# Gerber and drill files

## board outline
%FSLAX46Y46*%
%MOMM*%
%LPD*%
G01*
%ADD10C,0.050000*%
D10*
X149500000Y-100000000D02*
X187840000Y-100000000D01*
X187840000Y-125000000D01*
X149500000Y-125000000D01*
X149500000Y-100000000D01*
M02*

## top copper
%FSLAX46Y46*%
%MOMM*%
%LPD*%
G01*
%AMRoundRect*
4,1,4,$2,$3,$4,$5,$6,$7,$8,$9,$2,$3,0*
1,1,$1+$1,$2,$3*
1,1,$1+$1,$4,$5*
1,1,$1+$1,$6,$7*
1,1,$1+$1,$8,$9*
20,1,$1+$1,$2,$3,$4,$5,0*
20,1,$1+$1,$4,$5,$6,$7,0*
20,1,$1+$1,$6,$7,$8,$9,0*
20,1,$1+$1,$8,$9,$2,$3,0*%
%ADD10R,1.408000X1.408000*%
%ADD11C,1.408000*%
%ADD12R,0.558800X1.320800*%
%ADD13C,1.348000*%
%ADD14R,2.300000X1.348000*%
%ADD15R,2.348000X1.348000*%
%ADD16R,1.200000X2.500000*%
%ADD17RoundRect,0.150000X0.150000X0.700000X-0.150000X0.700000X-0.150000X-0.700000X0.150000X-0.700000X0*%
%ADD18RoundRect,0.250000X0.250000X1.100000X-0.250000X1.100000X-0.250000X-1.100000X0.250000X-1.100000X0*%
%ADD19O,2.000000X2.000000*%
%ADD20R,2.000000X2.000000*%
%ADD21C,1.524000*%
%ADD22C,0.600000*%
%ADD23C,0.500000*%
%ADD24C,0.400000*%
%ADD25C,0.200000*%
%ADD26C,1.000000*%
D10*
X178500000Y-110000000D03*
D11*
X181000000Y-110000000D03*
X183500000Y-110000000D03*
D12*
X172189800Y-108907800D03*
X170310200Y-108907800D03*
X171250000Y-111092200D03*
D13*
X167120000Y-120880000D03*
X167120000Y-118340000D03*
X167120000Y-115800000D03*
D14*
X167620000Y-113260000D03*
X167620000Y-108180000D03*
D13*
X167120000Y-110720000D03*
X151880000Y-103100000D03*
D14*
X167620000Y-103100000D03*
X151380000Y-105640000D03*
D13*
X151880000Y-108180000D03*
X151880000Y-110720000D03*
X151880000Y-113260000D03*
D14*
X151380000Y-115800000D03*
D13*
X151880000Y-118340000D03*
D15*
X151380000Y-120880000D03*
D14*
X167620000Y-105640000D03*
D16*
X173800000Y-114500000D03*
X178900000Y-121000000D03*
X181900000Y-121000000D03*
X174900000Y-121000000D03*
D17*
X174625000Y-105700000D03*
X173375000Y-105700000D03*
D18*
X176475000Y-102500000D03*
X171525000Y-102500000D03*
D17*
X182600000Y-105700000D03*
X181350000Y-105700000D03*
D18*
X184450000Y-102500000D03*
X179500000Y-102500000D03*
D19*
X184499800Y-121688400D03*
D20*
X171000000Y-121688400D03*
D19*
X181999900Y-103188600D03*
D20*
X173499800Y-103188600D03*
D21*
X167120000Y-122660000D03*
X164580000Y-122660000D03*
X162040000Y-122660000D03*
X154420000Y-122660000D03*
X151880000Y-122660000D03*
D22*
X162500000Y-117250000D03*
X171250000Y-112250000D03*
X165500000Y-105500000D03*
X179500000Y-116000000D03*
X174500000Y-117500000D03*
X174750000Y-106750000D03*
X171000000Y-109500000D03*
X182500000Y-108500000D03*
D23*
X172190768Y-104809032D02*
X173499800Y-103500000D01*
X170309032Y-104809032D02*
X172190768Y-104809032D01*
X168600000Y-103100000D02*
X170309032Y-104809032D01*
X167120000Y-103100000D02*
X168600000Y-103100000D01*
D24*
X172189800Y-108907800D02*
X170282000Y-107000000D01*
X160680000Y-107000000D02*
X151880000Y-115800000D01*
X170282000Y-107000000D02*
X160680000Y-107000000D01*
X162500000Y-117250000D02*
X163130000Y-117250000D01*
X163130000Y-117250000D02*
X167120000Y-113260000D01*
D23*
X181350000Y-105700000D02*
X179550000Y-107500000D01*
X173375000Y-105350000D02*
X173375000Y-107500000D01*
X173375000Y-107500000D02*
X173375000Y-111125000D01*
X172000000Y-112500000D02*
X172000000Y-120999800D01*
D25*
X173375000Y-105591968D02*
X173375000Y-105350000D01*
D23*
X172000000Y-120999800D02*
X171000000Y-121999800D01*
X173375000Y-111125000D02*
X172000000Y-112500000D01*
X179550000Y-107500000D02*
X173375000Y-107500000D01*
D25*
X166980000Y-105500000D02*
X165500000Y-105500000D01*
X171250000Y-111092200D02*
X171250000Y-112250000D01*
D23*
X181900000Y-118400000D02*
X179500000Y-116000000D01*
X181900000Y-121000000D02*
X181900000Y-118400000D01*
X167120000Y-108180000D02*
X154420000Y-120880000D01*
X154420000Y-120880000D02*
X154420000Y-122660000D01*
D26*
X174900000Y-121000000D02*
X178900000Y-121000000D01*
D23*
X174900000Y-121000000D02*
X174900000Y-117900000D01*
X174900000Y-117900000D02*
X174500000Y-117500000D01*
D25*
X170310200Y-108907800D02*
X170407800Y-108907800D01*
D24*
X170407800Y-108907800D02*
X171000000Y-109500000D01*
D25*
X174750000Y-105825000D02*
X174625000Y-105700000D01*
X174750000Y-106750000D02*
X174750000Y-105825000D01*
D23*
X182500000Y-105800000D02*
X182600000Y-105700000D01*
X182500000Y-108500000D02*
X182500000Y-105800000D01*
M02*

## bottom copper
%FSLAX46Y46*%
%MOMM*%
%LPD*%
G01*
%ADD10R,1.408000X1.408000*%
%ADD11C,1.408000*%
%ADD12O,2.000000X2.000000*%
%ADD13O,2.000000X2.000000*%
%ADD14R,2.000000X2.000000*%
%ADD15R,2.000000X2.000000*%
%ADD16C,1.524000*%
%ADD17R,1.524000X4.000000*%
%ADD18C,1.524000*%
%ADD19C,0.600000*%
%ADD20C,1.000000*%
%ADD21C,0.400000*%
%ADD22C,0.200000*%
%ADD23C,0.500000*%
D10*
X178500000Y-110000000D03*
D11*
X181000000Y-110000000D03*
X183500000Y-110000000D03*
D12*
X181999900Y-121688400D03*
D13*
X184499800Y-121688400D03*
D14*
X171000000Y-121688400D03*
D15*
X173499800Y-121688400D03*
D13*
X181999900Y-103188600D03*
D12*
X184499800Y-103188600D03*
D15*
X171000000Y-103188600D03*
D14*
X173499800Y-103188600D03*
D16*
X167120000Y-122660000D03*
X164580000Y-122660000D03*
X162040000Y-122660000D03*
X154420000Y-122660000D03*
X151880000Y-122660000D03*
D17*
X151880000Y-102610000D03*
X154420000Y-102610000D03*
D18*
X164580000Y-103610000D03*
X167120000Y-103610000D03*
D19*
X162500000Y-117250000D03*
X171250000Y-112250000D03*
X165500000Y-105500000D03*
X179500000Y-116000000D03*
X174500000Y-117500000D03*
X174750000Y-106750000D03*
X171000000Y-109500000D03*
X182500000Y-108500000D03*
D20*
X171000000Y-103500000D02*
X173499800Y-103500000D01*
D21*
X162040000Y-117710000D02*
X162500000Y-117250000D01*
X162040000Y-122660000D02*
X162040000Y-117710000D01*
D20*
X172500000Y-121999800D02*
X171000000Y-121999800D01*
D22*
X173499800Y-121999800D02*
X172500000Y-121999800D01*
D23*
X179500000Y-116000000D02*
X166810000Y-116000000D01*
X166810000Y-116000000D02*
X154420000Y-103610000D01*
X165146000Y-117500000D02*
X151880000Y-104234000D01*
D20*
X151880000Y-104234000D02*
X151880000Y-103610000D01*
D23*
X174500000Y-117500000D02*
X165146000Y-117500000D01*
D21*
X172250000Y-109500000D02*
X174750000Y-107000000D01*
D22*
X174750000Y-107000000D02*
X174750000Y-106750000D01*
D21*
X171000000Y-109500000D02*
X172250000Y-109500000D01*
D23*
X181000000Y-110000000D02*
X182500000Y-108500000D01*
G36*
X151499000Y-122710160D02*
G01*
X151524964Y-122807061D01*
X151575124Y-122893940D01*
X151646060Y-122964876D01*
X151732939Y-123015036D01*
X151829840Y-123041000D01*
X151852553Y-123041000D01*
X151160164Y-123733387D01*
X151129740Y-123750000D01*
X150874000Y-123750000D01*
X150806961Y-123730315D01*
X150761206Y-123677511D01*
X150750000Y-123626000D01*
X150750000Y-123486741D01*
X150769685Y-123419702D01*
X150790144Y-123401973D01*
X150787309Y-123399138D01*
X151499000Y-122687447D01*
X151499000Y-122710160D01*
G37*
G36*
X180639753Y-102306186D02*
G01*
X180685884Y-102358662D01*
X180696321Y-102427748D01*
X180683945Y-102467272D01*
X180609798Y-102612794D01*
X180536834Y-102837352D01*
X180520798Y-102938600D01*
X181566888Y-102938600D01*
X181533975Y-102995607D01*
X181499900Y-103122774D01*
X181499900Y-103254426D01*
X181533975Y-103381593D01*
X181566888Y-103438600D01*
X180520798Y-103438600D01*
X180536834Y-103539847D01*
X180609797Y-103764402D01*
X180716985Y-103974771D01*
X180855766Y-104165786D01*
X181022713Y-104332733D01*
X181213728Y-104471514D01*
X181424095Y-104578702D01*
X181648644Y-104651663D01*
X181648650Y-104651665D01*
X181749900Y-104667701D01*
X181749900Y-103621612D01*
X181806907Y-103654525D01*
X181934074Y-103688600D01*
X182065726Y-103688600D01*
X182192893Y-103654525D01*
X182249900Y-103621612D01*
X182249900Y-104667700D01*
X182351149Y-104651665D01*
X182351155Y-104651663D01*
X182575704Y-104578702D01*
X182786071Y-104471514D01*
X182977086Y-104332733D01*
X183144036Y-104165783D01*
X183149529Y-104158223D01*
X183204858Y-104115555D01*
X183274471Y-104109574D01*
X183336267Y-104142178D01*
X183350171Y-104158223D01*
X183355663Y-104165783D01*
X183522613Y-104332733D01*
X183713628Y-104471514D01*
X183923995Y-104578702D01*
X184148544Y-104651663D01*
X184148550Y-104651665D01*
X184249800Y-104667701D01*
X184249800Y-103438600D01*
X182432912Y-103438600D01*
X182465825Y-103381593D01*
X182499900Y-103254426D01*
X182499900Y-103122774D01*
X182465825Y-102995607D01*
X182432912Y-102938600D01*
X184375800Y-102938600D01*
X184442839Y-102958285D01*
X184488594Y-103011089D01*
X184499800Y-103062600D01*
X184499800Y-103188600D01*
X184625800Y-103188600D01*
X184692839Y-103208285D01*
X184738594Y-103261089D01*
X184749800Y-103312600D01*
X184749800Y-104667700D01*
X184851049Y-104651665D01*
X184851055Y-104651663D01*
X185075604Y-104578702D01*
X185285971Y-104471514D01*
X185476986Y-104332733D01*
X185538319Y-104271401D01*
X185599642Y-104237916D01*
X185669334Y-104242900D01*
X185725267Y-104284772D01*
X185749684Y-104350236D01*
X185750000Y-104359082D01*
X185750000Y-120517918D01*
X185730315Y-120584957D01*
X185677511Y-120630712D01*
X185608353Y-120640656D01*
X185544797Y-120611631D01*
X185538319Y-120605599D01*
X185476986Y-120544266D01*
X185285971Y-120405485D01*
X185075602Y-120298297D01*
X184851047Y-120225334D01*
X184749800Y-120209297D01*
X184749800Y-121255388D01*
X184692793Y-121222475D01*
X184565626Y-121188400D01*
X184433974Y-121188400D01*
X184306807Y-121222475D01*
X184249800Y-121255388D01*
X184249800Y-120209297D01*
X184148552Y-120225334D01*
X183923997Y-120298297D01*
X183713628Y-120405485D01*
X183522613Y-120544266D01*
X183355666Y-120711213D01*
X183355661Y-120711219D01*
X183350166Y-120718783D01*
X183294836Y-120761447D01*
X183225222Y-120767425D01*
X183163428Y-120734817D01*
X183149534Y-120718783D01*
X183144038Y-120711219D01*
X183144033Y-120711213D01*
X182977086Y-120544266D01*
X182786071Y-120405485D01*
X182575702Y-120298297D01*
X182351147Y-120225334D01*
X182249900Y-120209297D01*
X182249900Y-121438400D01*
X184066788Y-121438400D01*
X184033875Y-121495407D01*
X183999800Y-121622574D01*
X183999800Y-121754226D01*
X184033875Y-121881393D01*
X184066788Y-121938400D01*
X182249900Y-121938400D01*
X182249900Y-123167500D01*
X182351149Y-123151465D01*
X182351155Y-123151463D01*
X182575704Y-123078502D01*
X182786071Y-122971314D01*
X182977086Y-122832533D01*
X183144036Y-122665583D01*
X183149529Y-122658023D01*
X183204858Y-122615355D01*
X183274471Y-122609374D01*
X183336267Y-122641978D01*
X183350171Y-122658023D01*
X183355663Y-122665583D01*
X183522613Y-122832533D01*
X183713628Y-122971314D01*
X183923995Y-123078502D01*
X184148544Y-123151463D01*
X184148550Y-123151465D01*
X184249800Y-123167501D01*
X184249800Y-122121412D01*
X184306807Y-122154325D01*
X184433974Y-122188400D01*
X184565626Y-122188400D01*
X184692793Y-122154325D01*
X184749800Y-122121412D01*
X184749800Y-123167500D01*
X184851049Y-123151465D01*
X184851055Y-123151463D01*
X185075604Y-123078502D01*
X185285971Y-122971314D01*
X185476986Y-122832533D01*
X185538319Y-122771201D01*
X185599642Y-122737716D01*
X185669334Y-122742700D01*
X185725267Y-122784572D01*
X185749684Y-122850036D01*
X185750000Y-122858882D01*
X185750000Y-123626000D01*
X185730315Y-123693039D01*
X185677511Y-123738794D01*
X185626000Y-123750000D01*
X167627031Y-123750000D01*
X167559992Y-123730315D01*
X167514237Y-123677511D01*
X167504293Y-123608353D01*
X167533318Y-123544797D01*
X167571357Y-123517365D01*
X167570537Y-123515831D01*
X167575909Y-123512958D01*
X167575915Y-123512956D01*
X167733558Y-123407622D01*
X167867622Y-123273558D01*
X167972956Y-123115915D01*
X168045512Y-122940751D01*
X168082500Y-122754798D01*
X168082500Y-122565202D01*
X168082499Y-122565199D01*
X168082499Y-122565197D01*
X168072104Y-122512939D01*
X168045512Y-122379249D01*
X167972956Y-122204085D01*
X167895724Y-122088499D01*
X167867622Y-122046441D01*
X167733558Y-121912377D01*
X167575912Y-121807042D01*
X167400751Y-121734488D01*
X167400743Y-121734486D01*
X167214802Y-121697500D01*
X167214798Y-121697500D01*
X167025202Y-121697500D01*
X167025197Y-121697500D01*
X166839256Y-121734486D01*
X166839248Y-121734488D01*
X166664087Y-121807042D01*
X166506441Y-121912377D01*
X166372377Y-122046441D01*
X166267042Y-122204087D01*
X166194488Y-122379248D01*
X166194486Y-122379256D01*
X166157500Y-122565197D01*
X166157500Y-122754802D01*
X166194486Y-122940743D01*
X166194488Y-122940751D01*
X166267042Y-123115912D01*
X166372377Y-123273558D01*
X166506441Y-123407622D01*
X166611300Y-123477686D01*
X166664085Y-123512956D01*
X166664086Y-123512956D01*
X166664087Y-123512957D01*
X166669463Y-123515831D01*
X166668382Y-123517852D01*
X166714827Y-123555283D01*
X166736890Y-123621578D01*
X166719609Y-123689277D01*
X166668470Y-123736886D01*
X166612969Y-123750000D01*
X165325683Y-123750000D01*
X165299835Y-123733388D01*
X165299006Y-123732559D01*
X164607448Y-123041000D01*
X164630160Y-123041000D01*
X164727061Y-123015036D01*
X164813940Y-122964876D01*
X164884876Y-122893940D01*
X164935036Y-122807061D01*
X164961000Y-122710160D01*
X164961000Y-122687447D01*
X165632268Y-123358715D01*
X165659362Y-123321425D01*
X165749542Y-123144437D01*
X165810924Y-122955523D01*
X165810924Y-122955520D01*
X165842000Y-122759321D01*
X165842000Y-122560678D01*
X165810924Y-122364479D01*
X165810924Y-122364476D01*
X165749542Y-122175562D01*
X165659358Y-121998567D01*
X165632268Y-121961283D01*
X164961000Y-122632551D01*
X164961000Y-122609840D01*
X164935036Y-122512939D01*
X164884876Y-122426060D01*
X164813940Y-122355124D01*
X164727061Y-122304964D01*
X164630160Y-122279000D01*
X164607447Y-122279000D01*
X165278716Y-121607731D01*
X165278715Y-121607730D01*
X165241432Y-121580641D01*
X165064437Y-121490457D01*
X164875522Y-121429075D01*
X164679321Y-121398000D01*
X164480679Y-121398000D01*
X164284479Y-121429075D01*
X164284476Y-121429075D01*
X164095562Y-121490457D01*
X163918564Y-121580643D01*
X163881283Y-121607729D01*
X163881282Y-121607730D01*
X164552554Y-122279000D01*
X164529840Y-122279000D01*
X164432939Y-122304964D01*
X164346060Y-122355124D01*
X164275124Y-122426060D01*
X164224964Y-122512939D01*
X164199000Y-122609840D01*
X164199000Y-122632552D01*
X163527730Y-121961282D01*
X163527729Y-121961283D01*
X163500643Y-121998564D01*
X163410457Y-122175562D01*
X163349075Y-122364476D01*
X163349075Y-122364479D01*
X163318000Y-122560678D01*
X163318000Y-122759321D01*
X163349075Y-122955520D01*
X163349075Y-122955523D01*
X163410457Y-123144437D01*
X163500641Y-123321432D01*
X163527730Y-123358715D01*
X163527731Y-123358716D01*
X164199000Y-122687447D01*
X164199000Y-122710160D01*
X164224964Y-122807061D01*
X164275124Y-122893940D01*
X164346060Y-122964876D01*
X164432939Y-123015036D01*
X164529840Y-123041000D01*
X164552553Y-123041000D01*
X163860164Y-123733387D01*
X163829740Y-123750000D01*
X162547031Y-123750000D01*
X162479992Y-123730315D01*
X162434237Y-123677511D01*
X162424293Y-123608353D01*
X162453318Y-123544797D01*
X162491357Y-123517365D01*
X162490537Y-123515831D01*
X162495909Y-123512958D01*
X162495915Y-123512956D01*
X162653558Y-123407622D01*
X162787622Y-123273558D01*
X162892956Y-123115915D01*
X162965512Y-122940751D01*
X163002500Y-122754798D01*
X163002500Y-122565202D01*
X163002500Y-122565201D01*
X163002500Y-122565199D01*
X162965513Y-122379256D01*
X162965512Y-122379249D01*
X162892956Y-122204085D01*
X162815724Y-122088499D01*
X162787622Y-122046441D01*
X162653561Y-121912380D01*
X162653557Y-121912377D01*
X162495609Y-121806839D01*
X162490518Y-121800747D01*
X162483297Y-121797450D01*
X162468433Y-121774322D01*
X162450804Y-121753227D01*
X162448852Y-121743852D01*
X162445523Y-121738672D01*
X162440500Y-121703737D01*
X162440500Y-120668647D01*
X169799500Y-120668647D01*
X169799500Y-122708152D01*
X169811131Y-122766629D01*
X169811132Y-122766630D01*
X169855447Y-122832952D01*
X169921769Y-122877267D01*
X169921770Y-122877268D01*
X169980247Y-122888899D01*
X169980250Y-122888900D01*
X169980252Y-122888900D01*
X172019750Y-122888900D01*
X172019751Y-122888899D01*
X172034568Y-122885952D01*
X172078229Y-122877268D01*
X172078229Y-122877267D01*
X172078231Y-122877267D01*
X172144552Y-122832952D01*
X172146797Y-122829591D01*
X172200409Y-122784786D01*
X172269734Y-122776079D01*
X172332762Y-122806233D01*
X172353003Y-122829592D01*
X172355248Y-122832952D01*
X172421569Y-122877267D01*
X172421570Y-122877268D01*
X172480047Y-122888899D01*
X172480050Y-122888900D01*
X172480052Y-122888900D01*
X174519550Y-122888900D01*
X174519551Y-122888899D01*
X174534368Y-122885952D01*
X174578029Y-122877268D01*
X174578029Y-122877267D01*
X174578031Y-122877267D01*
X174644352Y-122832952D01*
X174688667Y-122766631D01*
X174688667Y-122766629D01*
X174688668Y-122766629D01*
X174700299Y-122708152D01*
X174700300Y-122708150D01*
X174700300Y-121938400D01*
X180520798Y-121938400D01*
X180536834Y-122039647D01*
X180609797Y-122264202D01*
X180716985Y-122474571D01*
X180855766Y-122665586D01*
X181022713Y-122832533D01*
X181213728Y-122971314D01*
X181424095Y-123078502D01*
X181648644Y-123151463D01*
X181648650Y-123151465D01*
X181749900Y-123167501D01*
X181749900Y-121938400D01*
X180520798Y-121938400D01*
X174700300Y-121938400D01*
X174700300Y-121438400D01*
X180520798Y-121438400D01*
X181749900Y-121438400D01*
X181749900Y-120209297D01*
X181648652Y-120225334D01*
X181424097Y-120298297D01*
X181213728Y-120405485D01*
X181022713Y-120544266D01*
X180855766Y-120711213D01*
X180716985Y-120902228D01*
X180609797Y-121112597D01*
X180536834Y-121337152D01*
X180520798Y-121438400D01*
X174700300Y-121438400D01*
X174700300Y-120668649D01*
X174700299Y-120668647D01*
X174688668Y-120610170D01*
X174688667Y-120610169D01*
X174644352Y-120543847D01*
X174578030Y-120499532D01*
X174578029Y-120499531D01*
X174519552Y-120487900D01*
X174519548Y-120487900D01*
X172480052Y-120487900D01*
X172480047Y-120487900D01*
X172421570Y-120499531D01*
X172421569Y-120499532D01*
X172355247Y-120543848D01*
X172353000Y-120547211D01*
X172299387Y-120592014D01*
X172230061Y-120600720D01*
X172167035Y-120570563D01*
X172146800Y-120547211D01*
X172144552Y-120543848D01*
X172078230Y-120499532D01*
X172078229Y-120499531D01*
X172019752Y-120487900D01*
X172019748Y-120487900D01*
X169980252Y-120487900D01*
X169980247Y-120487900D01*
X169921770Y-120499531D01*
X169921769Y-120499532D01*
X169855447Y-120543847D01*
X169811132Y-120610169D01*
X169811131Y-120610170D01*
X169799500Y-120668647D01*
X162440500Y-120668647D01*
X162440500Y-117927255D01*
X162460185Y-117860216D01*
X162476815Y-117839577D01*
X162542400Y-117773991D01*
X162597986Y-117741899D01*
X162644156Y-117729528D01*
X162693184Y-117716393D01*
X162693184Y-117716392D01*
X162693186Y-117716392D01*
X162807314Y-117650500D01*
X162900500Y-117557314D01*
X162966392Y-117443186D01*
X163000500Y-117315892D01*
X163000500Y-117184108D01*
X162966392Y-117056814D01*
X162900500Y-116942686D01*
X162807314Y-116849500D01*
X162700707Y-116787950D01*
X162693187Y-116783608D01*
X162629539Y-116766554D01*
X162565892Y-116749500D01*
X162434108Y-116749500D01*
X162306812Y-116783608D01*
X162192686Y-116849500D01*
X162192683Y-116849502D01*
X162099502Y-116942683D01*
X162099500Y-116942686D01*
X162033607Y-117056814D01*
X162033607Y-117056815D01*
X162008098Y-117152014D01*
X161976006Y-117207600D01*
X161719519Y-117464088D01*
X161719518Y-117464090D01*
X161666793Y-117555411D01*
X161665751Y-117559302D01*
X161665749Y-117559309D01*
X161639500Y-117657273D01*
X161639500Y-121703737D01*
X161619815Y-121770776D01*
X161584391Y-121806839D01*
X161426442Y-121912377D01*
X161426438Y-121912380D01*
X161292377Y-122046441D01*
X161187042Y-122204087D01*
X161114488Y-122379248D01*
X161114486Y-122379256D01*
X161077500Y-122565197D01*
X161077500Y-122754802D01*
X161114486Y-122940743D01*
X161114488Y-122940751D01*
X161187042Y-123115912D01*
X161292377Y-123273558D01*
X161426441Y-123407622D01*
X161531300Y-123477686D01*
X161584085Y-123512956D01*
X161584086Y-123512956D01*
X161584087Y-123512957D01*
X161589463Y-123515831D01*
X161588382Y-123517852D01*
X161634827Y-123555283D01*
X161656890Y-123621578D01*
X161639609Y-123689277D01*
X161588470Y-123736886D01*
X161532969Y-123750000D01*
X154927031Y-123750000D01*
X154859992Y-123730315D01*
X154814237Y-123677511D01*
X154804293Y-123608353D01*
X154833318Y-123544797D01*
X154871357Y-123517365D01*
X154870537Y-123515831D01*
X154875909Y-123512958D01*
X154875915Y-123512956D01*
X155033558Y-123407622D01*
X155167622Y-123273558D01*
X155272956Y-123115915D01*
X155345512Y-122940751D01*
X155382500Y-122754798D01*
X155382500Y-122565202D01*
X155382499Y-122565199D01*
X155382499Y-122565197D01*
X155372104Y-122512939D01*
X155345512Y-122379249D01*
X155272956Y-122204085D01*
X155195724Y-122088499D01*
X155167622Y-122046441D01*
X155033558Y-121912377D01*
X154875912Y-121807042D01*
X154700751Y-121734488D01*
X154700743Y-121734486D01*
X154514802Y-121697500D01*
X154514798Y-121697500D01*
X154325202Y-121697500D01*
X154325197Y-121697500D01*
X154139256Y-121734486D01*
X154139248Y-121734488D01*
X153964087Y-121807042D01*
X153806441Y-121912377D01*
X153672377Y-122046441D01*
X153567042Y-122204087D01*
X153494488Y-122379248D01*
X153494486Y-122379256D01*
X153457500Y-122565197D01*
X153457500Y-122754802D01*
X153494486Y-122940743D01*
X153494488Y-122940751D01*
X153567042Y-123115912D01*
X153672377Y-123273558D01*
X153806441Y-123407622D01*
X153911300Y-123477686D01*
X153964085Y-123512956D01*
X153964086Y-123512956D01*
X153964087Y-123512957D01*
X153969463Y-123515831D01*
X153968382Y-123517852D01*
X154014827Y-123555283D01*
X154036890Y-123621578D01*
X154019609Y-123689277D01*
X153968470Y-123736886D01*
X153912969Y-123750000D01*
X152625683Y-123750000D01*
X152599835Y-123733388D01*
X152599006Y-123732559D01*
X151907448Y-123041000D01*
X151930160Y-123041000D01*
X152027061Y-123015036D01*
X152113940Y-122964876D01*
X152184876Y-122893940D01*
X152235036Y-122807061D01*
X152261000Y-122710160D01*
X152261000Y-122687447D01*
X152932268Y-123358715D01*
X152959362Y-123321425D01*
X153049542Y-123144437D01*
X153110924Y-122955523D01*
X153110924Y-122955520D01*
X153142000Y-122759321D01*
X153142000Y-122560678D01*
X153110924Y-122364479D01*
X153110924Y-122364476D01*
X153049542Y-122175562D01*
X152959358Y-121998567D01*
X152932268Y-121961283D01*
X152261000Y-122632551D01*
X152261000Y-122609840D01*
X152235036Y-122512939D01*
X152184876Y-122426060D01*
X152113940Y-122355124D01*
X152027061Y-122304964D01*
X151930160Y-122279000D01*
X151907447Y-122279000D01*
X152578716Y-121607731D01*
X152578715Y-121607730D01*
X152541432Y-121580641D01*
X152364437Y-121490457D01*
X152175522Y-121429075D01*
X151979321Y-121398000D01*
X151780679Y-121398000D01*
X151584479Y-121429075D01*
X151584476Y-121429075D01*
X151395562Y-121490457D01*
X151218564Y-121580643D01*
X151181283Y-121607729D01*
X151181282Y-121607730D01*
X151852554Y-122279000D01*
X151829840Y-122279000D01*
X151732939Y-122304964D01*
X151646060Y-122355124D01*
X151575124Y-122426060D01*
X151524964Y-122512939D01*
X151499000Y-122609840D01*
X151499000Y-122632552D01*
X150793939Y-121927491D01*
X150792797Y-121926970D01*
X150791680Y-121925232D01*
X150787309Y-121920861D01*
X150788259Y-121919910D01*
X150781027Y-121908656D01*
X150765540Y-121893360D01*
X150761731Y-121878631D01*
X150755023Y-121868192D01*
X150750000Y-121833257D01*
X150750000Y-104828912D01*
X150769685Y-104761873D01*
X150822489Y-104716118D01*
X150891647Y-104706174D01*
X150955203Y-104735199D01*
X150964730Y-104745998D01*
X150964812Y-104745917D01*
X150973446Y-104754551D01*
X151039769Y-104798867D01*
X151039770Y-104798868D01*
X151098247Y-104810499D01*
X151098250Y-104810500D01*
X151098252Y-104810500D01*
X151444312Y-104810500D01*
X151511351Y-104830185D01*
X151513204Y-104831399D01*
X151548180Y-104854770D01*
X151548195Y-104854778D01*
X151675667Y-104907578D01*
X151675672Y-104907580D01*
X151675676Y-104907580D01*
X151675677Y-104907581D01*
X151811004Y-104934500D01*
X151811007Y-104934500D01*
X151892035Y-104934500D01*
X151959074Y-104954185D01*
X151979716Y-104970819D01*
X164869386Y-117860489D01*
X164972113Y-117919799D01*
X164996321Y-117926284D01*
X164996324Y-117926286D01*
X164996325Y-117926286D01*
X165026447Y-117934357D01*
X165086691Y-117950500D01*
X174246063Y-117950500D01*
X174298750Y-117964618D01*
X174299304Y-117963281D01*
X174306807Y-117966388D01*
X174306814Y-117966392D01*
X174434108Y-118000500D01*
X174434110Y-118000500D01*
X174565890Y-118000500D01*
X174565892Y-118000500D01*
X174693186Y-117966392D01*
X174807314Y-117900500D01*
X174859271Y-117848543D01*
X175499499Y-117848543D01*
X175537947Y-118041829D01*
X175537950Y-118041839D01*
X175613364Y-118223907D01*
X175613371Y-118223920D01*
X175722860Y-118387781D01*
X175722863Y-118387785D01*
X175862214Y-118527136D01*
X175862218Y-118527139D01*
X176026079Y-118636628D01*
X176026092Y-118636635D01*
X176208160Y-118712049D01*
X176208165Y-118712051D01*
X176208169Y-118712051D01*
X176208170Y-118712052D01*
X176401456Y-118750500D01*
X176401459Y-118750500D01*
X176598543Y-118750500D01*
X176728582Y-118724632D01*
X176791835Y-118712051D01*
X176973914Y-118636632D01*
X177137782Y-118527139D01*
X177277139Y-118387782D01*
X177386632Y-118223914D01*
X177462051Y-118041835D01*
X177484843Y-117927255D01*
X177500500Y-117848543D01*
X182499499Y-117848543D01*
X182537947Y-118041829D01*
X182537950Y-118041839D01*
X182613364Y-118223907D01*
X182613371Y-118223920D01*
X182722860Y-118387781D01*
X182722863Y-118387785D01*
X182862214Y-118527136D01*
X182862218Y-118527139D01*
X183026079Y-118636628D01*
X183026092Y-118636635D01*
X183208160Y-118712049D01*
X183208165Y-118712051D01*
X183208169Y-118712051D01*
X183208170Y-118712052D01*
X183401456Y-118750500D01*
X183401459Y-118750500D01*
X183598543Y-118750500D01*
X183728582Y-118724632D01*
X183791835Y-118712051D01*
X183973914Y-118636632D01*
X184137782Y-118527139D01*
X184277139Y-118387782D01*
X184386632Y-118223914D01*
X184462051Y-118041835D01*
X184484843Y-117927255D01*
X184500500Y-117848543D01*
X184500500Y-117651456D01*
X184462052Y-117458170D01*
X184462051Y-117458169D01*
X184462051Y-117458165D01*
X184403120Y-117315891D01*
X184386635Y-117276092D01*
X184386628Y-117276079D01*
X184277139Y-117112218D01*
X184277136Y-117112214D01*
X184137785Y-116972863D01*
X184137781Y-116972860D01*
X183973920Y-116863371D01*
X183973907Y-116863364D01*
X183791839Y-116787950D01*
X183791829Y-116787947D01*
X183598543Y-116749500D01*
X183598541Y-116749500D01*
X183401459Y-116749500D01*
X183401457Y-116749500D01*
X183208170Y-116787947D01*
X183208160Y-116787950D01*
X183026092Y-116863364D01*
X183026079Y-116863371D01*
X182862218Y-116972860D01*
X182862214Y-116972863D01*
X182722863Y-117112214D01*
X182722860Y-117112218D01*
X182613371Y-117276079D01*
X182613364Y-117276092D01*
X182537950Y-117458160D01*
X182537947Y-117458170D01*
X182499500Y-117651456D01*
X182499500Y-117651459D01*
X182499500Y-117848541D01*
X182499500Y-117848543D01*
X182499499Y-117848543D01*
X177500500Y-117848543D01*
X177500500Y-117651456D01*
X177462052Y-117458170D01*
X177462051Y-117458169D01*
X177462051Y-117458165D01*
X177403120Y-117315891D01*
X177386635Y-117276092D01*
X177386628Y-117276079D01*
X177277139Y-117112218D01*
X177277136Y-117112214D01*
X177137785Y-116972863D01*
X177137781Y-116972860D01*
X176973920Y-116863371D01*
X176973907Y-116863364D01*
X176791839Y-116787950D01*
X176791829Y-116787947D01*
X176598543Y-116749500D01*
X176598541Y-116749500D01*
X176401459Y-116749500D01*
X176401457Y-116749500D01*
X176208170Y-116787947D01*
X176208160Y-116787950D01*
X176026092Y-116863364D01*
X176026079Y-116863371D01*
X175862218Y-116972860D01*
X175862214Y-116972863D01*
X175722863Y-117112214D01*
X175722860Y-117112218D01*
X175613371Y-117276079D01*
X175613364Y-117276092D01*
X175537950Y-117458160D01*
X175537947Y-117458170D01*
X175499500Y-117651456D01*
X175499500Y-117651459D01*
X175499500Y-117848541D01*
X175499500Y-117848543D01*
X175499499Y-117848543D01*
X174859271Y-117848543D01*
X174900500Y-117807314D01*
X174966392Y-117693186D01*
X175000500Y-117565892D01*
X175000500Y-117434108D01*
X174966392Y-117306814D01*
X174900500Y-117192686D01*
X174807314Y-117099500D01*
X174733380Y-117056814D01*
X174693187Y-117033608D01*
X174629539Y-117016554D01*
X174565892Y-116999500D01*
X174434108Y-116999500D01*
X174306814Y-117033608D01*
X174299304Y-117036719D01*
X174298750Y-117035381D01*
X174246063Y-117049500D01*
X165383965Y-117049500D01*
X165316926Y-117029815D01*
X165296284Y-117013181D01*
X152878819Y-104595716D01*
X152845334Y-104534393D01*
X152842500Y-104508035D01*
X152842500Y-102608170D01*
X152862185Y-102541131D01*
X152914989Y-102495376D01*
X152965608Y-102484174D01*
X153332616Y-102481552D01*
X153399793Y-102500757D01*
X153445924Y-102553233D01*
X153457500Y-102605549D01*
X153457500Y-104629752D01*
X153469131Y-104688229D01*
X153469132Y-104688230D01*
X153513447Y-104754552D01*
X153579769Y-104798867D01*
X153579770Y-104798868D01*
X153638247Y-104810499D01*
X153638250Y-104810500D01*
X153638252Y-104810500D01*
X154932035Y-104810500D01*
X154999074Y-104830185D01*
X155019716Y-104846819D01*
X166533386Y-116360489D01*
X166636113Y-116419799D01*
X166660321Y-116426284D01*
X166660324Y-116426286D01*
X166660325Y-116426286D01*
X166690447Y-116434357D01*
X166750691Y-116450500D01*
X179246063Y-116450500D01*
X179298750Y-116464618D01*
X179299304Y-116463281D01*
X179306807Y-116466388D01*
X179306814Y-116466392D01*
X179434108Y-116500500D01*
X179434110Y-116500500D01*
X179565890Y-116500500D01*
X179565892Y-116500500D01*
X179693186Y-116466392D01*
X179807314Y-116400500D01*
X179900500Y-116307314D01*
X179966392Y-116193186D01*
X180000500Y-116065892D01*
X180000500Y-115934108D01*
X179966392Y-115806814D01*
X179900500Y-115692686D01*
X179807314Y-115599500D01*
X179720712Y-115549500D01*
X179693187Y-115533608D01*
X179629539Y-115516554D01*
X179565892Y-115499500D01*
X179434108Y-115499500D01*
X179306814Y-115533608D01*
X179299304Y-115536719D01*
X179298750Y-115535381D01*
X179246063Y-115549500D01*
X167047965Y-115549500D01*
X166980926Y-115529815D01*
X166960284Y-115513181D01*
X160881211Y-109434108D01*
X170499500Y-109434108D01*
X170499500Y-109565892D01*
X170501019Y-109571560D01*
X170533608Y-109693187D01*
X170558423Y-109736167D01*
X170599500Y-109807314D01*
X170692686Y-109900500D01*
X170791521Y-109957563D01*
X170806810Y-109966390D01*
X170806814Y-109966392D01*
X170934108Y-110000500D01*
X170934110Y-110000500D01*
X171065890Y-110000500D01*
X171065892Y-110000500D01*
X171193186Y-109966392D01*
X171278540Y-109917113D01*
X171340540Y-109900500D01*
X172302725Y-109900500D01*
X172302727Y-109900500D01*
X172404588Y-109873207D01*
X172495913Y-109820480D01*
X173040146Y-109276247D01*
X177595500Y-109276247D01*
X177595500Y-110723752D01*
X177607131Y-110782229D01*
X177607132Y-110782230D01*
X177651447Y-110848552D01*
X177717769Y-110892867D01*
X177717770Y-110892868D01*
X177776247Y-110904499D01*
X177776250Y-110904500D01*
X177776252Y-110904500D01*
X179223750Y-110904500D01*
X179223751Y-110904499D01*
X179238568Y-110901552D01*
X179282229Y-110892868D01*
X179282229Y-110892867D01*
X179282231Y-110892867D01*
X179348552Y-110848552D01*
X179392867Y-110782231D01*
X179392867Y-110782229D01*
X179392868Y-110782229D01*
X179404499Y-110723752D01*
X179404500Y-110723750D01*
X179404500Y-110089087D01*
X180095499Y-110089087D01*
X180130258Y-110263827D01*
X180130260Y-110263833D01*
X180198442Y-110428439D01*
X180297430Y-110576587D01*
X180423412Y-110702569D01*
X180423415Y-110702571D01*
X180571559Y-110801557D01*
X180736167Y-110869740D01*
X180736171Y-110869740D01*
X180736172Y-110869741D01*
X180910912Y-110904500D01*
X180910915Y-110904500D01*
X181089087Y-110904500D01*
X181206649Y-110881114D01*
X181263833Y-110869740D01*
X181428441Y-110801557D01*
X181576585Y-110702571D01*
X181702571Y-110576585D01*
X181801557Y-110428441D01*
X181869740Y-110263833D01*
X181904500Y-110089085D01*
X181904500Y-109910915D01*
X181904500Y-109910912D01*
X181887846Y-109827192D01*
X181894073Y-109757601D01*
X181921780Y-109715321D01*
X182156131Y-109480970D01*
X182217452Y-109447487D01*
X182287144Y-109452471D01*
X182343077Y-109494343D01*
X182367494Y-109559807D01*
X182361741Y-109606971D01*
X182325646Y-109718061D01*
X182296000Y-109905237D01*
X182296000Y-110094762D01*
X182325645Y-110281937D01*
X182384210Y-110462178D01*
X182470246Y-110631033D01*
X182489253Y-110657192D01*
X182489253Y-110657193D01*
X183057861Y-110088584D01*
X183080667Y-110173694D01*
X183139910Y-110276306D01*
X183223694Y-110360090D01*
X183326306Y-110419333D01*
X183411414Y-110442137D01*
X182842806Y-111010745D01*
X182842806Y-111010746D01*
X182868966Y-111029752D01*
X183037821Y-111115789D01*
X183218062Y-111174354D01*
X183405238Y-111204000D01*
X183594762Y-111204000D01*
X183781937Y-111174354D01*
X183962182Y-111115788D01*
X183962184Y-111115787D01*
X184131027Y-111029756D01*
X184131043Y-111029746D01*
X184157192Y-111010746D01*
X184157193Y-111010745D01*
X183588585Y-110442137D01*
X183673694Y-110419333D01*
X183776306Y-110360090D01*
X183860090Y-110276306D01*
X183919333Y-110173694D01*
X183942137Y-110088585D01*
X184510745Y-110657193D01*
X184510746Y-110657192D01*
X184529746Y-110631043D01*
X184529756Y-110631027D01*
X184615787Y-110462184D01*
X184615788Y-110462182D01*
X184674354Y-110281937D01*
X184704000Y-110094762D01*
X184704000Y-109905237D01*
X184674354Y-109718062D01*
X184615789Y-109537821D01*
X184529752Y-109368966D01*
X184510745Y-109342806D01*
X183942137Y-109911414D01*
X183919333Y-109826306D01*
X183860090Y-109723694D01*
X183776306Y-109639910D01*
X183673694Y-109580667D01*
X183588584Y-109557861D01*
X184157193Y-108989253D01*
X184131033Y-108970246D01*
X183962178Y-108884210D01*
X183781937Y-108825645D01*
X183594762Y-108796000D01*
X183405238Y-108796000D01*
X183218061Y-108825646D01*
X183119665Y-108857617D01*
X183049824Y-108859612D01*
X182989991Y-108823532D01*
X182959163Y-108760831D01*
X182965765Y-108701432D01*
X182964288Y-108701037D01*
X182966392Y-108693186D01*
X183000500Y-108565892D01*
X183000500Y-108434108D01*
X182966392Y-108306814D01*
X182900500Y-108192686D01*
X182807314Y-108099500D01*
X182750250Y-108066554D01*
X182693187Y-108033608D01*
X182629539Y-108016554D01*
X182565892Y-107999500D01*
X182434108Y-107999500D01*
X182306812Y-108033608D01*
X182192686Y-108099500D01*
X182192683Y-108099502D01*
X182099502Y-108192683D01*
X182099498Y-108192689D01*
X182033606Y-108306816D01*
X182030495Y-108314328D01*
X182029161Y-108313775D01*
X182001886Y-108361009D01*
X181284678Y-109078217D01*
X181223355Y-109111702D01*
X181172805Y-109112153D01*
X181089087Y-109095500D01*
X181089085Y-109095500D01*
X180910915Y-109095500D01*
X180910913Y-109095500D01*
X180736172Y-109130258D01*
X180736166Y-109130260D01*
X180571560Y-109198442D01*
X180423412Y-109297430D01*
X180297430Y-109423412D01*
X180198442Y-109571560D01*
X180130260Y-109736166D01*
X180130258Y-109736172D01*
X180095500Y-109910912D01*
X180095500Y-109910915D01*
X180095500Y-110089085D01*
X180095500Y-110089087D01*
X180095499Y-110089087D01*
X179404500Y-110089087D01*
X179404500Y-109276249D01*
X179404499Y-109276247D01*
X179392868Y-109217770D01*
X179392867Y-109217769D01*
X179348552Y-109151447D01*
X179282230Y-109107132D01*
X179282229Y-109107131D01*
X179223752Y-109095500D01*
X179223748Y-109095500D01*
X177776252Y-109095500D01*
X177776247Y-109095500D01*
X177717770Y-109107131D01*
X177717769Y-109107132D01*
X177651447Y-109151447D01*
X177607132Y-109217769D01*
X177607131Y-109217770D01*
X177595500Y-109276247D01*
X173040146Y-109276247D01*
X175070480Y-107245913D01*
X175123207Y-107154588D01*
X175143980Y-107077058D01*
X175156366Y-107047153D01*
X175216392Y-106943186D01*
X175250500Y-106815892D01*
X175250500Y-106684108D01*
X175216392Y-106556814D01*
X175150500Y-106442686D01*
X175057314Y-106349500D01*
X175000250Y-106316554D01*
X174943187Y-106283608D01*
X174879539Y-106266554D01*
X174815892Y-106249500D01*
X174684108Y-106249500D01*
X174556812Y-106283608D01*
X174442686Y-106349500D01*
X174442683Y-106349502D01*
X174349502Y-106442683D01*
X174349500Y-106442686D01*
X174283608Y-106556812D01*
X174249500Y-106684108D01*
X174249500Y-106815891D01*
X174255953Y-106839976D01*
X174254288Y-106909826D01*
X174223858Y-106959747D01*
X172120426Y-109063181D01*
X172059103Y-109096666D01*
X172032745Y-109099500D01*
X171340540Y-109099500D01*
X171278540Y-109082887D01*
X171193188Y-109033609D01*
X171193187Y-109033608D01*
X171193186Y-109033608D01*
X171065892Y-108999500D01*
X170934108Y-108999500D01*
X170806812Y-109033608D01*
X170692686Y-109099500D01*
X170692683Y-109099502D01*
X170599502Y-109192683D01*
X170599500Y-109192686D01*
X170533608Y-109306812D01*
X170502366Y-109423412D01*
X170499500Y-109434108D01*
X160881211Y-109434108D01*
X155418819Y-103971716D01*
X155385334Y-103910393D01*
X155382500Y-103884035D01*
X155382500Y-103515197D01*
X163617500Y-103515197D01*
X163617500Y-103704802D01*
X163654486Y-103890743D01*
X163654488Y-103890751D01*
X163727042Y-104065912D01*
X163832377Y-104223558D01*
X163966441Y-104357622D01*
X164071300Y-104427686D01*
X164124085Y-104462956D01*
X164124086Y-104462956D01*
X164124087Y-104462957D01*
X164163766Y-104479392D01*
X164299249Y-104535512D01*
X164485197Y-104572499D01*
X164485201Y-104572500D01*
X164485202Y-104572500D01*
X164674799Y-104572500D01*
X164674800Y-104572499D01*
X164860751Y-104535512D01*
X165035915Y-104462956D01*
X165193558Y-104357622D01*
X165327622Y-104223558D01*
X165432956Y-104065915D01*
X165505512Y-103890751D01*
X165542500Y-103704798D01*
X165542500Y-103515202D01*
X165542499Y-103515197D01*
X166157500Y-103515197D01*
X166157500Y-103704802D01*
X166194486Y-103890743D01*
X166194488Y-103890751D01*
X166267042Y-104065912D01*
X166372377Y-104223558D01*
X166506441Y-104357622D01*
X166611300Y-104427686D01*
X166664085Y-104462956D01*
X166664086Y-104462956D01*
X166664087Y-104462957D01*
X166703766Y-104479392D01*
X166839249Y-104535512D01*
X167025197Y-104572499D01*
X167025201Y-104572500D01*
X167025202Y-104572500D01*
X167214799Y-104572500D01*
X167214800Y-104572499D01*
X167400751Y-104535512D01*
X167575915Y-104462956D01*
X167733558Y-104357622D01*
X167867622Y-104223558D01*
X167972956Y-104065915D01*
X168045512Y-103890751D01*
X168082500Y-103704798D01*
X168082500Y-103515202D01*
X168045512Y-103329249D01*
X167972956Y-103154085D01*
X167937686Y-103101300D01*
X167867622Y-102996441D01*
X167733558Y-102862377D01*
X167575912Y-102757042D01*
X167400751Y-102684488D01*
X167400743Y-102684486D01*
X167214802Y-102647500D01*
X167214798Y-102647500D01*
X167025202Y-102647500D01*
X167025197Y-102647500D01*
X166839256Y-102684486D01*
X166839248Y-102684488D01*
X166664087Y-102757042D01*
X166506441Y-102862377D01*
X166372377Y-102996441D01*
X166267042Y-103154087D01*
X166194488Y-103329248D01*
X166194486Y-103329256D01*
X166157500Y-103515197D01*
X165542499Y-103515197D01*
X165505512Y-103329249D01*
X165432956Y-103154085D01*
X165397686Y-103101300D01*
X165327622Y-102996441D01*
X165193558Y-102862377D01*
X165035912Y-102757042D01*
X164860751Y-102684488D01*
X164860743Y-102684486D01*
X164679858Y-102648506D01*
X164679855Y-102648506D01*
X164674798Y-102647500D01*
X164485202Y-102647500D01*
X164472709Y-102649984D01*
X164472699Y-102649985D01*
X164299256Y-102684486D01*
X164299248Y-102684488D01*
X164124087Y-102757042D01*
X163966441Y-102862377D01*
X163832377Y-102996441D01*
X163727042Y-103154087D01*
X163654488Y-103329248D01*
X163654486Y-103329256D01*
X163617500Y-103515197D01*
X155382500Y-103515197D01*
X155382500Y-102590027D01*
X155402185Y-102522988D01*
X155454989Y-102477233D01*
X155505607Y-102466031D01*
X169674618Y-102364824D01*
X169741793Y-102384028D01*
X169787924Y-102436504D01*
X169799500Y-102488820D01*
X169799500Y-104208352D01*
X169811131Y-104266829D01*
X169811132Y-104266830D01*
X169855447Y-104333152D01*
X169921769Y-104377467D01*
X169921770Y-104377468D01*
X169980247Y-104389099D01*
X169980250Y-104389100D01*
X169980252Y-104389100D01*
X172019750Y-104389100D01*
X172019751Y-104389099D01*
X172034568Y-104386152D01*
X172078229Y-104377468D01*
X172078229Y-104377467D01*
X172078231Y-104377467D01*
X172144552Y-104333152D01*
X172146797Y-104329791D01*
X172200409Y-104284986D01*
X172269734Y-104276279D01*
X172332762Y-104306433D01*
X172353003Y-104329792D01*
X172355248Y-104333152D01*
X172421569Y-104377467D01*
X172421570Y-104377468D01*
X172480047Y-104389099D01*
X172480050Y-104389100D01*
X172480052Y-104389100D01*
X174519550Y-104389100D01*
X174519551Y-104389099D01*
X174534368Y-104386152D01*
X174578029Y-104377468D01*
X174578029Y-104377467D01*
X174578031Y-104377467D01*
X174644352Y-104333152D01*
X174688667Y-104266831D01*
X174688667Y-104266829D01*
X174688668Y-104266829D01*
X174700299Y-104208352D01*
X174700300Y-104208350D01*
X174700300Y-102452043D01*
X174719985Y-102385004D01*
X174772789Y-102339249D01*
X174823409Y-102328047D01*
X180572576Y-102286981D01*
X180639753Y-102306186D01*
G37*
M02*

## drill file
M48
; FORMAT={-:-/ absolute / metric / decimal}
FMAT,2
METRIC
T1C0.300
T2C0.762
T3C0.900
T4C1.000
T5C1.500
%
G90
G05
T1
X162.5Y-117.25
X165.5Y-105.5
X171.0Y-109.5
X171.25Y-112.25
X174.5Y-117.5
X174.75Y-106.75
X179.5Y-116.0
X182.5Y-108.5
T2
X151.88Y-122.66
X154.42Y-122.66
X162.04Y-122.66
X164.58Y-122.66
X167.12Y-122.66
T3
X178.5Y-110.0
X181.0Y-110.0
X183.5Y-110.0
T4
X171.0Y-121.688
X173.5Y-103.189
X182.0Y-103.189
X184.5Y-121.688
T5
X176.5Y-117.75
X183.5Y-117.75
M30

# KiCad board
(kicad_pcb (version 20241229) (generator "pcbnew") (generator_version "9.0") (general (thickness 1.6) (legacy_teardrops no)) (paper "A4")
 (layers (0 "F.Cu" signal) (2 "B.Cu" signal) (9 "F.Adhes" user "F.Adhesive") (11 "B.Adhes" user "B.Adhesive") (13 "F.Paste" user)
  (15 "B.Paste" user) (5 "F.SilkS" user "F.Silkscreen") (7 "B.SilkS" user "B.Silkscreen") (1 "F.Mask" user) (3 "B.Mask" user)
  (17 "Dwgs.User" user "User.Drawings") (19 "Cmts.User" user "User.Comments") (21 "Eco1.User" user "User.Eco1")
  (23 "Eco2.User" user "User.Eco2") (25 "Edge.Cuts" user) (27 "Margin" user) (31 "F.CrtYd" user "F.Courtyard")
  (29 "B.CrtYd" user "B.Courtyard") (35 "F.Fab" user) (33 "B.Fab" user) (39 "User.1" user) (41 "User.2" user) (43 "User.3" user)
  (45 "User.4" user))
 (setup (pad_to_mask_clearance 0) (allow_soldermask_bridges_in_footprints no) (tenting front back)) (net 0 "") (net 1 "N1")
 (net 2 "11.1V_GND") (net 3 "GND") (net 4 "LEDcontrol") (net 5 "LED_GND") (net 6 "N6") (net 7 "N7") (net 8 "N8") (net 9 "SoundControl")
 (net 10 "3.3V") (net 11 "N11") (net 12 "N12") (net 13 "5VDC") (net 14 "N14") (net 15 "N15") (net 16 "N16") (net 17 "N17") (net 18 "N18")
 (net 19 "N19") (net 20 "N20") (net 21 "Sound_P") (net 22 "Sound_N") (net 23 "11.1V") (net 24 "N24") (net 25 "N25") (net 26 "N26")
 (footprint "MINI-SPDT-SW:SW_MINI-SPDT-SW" (layer "F.Cu") (at 181 110)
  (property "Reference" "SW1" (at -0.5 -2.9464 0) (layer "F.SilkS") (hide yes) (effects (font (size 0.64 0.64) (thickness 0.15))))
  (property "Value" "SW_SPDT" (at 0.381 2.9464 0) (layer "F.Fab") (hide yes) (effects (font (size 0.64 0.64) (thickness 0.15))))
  (pad "1" thru_hole rect (at -2.5 0) (size 1.408 1.408) (drill 0.9) (layers "*.Cu" "*.Mask") (remove_unused_layers no) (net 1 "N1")
   (solder_mask_margin 0.102))
  (pad "2" thru_hole circle (at 0 0) (size 1.408 1.408) (drill 0.9) (layers "*.Cu" "*.Mask") (remove_unused_layers no) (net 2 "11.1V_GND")
   (solder_mask_margin 0.102))
  (pad "3" thru_hole circle (at 2.5 0) (size 1.408 1.408) (drill 0.9) (layers "*.Cu" "*.Mask") (remove_unused_layers no) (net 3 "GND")
   (solder_mask_margin 0.102)))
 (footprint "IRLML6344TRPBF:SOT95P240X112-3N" (layer "F.Cu") (at 171.25 110 -90)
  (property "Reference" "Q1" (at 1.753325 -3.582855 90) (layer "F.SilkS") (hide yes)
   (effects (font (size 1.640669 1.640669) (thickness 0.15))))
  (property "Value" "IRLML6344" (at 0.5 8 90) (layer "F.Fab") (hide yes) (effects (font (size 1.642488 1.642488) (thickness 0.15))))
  (pad "1" smd rect (at -1.0922 -0.9398 270) (size 1.3208 0.5588) (layers "F.Cu" "F.Mask" "F.Paste") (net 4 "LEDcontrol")
   (solder_mask_margin 0.102))
  (pad "2" smd rect (at -1.0922 0.9398 270) (size 1.3208 0.5588) (layers "F.Cu" "F.Mask" "F.Paste") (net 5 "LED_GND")
   (solder_mask_margin 0.102))
  (pad "3" smd rect (at 1.0922 0 270) (size 1.3208 0.5588) (layers "F.Cu" "F.Mask" "F.Paste") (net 3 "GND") (solder_mask_margin 0.102)))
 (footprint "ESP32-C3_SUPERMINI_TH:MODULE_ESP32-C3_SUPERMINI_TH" (layer "F.Cu") (at 159.5 113)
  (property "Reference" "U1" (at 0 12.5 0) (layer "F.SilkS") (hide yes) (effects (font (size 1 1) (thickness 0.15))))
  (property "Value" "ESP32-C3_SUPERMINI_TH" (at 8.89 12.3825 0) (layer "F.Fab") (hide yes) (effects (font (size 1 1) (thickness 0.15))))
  (pad "0" smd circle (at 7.62 7.88) (size 1.348 1.348) (layers "F.Cu" "F.Mask" "F.Paste") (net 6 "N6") (solder_mask_margin 0.102))
  (pad "1" smd circle (at 7.62 5.34) (size 1.348 1.348) (layers "F.Cu" "F.Mask" "F.Paste") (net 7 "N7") (solder_mask_margin 0.102))
  (pad "2" smd circle (at 7.62 2.8) (size 1.348 1.348) (layers "F.Cu" "F.Mask" "F.Paste") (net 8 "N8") (solder_mask_margin 0.102))
  (pad "3" smd rect (at 7.62 0.26) (size 2.3 1.348) (drill (offset 0.5 0)) (layers "F.Cu" "F.Mask" "F.Paste") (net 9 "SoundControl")
   (solder_mask_margin 0.102))
  (pad "3.3" smd rect (at 7.62 -4.82) (size 2.3 1.348) (drill (offset 0.5 0)) (layers "F.Cu" "F.Mask" "F.Paste") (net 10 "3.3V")
   (solder_mask_margin 0.102))
  (pad "4" smd circle (at 7.62 -2.28) (size 1.348 1.348) (layers "F.Cu" "F.Mask" "F.Paste") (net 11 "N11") (solder_mask_margin 0.102))
  (pad "5" smd circle (at -7.62 -9.9) (size 1.348 1.348) (layers "F.Cu" "F.Mask" "F.Paste") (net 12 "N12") (solder_mask_margin 0.102))
  (pad "5V" smd rect (at 7.62 -9.9) (size 2.3 1.348) (drill (offset 0.5 0)) (layers "F.Cu" "F.Mask" "F.Paste") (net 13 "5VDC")
   (solder_mask_margin 0.102))
  (pad "6" smd rect (at -7.62 -7.36) (size 2.3 1.348) (drill (offset -0.5 0)) (layers "F.Cu" "F.Mask" "F.Paste") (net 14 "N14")
   (solder_mask_margin 0.102))
  (pad "7" smd circle (at -7.62 -4.82) (size 1.348 1.348) (layers "F.Cu" "F.Mask" "F.Paste") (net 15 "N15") (solder_mask_margin 0.102))
  (pad "8" smd circle (at -7.62 -2.28) (size 1.348 1.348) (layers "F.Cu" "F.Mask" "F.Paste") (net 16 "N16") (solder_mask_margin 0.102))
  (pad "9" smd circle (at -7.62 0.26) (size 1.348 1.348) (layers "F.Cu" "F.Mask" "F.Paste") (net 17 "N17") (solder_mask_margin 0.102))
  (pad "10" smd rect (at -7.62 2.8) (size 2.3 1.348) (drill (offset -0.5 0)) (layers "F.Cu" "F.Mask" "F.Paste") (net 4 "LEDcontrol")
   (solder_mask_margin 0.102))
  (pad "20" smd circle (at -7.62 5.34) (size 1.348 1.348) (layers "F.Cu" "F.Mask" "F.Paste") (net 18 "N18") (solder_mask_margin 0.102))
  (pad "21" smd rect (at -7.62 7.88) (size 2.348 1.348) (drill (offset -0.5 0)) (layers "F.Cu" "F.Mask" "F.Paste") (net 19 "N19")
   (solder_mask_margin 0.102))
  (pad "G" smd rect (at 7.62 -7.36) (size 2.3 1.348) (drill (offset 0.5 0)) (layers "F.Cu" "F.Mask" "F.Paste") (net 3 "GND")
   (solder_mask_margin 0.102)))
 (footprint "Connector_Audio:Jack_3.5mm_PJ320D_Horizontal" (layer "F.Cu") (at 178.725 117.75 180)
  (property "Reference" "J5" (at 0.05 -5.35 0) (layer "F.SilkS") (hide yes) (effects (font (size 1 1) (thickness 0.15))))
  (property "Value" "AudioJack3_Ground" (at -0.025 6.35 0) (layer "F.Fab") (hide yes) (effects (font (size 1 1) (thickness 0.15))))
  (pad "" np_thru_hole circle (at -4.775 0 180) (size 1.5 1.5) (drill 1.5) (layers "*.Cu" "*.Mask"))
  (pad "" np_thru_hole circle (at 2.225 0 180) (size 1.5 1.5) (drill 1.5) (layers "*.Cu" "*.Mask"))
  (pad "G" smd rect (at 4.925 3.25 180) (size 1.2 2.5) (layers "F.Cu" "F.Mask" "F.Paste") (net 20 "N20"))
  (pad "R" smd rect (at -0.175 -3.25 180) (size 1.2 2.5) (layers "F.Cu" "F.Mask" "F.Paste") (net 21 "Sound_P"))
  (pad "S" smd rect (at -3.175 -3.25 180) (size 1.2 2.5) (layers "F.Cu" "F.Mask" "F.Paste") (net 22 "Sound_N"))
  (pad "T" smd rect (at 3.825 -3.25 180) (size 1.2 2.5) (layers "F.Cu" "F.Mask" "F.Paste") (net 21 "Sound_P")))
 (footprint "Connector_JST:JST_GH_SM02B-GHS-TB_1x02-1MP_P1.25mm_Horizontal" (layer "F.Cu") (at 174 103.85 180)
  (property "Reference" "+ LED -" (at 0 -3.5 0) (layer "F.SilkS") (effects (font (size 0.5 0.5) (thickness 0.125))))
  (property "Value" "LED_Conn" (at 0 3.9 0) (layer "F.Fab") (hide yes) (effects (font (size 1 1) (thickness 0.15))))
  (pad "1" smd roundrect (at -0.625 -1.85 180) (size 0.6 1.7) (layers "F.Cu" "F.Mask" "F.Paste") (roundrect_rratio 0.25) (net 5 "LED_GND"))
  (pad "2" smd roundrect (at 0.625 -1.85 180) (size 0.6 1.7) (layers "F.Cu" "F.Mask" "F.Paste") (roundrect_rratio 0.25) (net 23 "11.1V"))
  (pad "MP" smd roundrect (at -2.475 1.35 180) (size 1 2.7) (layers "F.Cu" "F.Mask" "F.Paste") (roundrect_rratio 0.25))
  (pad "MP" smd roundrect (at 2.475 1.35 180) (size 1 2.7) (layers "F.Cu" "F.Mask" "F.Paste") (roundrect_rratio 0.25)))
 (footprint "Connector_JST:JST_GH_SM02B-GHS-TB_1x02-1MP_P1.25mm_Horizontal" (layer "F.Cu") (at 181.975 103.85 180)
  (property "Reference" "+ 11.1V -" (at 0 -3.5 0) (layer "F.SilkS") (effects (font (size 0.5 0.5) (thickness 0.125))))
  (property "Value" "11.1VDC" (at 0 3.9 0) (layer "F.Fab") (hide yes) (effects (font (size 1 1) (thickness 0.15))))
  (pad "1" smd roundrect (at -0.625 -1.85 180) (size 0.6 1.7) (layers "F.Cu" "F.Mask" "F.Paste") (roundrect_rratio 0.25) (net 2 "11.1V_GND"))
  (pad "2" smd roundrect (at 0.625 -1.85 180) (size 0.6 1.7) (layers "F.Cu" "F.Mask" "F.Paste") (roundrect_rratio 0.25) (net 23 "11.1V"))
  (pad "MP" smd roundrect (at -2.475 1.35 180) (size 1 2.7) (layers "F.Cu" "F.Mask" "F.Paste") (roundrect_rratio 0.25))
  (pad "MP" smd roundrect (at 2.475 1.35 180) (size 1 2.7) (layers "F.Cu" "F.Mask" "F.Paste") (roundrect_rratio 0.25)))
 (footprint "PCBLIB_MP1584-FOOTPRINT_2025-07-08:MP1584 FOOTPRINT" (layer "B.Cu") (at 169.2499 123.4385 90)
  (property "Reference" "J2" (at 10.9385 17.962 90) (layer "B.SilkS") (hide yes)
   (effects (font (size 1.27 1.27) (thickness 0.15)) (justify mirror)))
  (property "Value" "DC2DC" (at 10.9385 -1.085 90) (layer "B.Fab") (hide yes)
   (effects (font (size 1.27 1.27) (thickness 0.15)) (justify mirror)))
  (pad "1" smd oval (at 1.7501 12.75 90) (size 2 2) (layers "B.Cu" "B.Mask" "B.Paste") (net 3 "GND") (solder_mask_margin 0.0508)
   (solder_paste_margin 0) (thermal_bridge_angle 0))
  (pad "1" thru_hole oval (at 1.7501 15.2499 90) (size 2 2) (drill 1) (layers "*.Cu" "*.Mask") (remove_unused_layers no) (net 3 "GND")
   (solder_mask_margin 0.0508) (solder_paste_margin 0) (thermal_bridge_angle 0))
  (pad "2" thru_hole rect (at 1.7501 1.7501 90) (size 2 2) (drill 1) (layers "*.Cu" "*.Mask") (remove_unused_layers no) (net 23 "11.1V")
   (solder_mask_margin 0.0508) (solder_paste_margin 0) (thermal_bridge_angle 0))
  (pad "2" smd rect (at 1.7501 4.2499 90) (size 2 2) (layers "B.Cu" "B.Mask" "B.Paste") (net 23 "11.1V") (solder_mask_margin 0.0508)
   (solder_paste_margin 0) (thermal_bridge_angle 0))
  (pad "3" thru_hole oval (at 20.2499 12.75 90) (size 2 2) (drill 1) (layers "*.Cu" "*.Mask") (remove_unused_layers no) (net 3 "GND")
   (solder_mask_margin 0.0508) (solder_paste_margin 0) (thermal_bridge_angle 0))
  (pad "3" smd oval (at 20.2499 15.2499 90) (size 2 2) (layers "B.Cu" "B.Mask" "B.Paste") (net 3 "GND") (solder_mask_margin 0.0508)
   (solder_paste_margin 0) (thermal_bridge_angle 0))
  (pad "4" smd rect (at 20.2499 1.7501 90) (size 2 2) (layers "B.Cu" "B.Mask" "B.Paste") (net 13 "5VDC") (solder_mask_margin 0.0508)
   (solder_paste_margin 0) (thermal_bridge_angle 0))
  (pad "4" thru_hole rect (at 20.2499 4.2499 90) (size 2 2) (drill 1) (layers "*.Cu" "*.Mask") (remove_unused_layers no) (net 13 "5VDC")
   (solder_mask_margin 0.0508) (solder_paste_margin 0) (thermal_bridge_angle 0)))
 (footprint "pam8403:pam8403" (layer "B.Cu") (at 159.5 112.5 180)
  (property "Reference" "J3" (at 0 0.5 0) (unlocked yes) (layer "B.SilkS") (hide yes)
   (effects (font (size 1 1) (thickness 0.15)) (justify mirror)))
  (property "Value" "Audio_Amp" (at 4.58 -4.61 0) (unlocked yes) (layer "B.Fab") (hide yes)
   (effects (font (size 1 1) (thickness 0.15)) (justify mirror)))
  (pad "1" thru_hole circle (at -7.62 -10.16 180) (size 1.524 1.524) (drill 0.762) (layers "*.Cu" "*.Mask") (remove_unused_layers no)
   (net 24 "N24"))
  (pad "2" thru_hole circle (at -5.08 -10.16 180) (size 1.524 1.524) (drill 0.762) (layers "*.Cu" "*.Mask") (remove_unused_layers no)
   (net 3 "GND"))
  (pad "3" thru_hole circle (at -2.54 -10.16 180) (size 1.524 1.524) (drill 0.762) (layers "*.Cu" "*.Mask") (remove_unused_layers no)
   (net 9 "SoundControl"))
  (pad "4" thru_hole circle (at 5.08 -10.16 180) (size 1.524 1.524) (drill 0.762) (layers "*.Cu" "*.Mask") (remove_unused_layers no)
   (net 10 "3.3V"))
  (pad "5" thru_hole circle (at 7.62 -10.16 180) (size 1.524 1.524) (drill 0.762) (layers "*.Cu" "*.Mask") (remove_unused_layers no)
   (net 3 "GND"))
  (pad "6" smd rect (at 7.62 8.89 180) (size 1.524 4) (drill (offset 0 1)) (layers "B.Cu" "B.Mask" "B.Paste") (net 21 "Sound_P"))
  (pad "7" smd rect (at 5.08 8.89 180) (size 1.524 4) (drill (offset 0 1)) (layers "B.Cu" "B.Mask" "B.Paste") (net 22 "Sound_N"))
  (pad "8" smd circle (at -5.08 8.89 180) (size 1.524 1.524) (layers "B.Cu" "B.Mask" "B.Paste") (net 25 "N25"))
  (pad "9" smd circle (at -7.62 8.89 180) (size 1.524 1.524) (layers "B.Cu" "B.Mask" "B.Paste") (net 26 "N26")))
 (gr_rect (start 149.5 100) (end 187.84 125) (stroke (width 0.05) (type default)) (fill no) (layer "Edge.Cuts"))
 (segment (start 172.190768 104.809032) (end 173.4998 103.5) (width 0.5) (layer "F.Cu") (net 13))
 (segment (start 170.309032 104.809032) (end 172.190768 104.809032) (width 0.5) (layer "F.Cu") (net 13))
 (segment (start 168.6 103.1) (end 170.309032 104.809032) (width 0.5) (layer "F.Cu") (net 13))
 (segment (start 167.12 103.1) (end 168.6 103.1) (width 0.5) (layer "F.Cu") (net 13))
 (segment (start 171 103.5) (end 173.4998 103.5) (width 1) (layer "B.Cu") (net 13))
 (segment (start 172.1898 108.9078) (end 170.282 107) (width 0.4) (layer "F.Cu") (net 4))
 (segment (start 160.68 107) (end 151.88 115.8) (width 0.4) (layer "F.Cu") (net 4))
 (segment (start 170.282 107) (end 160.68 107) (width 0.4) (layer "F.Cu") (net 4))
 (segment (start 162.5 117.25) (end 163.13 117.25) (width 0.4) (layer "F.Cu") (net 9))
 (segment (start 163.13 117.25) (end 167.12 113.26) (width 0.4) (layer "F.Cu") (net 9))
 (via (at 162.5 117.25) (size 0.6) (drill 0.3) (layers "F.Cu" "B.Cu") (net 9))
 (segment (start 162.04 117.71) (end 162.5 117.25) (width 0.4) (layer "B.Cu") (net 9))
 (segment (start 162.04 122.66) (end 162.04 117.71) (width 0.4) (layer "B.Cu") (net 9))
 (segment (start 181.35 105.7) (end 179.55 107.5) (width 0.5) (layer "F.Cu") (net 23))
 (segment (start 173.375 105.35) (end 173.375 107.5) (width 0.5) (layer "F.Cu") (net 23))
 (segment (start 173.375 107.5) (end 173.375 111.125) (width 0.5) (layer "F.Cu") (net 23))
 (segment (start 172 112.5) (end 172 120.9998) (width 0.5) (layer "F.Cu") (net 23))
 (segment (start 173.375 105.591968) (end 173.375 105.35) (width 0.2) (layer "F.Cu") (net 23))
 (segment (start 172 120.9998) (end 171 121.9998) (width 0.5) (layer "F.Cu") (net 23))
 (segment (start 173.375 111.125) (end 172 112.5) (width 0.5) (layer "F.Cu") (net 23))
 (segment (start 179.55 107.5) (end 173.375 107.5) (width 0.5) (layer "F.Cu") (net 23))
 (segment (start 172.5 121.9998) (end 171 121.9998) (width 1) (layer "B.Cu") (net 23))
 (segment (start 173.4998 121.9998) (end 172.5 121.9998) (width 0.2) (layer "B.Cu") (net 23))
 (segment (start 166.98 105.5) (end 165.5 105.5) (width 0.2) (layer "F.Cu") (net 3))
 (segment (start 171.25 111.0922) (end 171.25 112.25) (width 0.2) (layer "F.Cu") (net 3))
 (via (at 171.25 112.25) (size 0.6) (drill 0.3) (layers "F.Cu" "B.Cu") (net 3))
 (via (at 165.5 105.5) (size 0.6) (drill 0.3) (layers "F.Cu" "B.Cu") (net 3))
 (segment (start 181.9 118.4) (end 179.5 116) (width 0.5) (layer "F.Cu") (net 22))
 (segment (start 181.9 121) (end 181.9 118.4) (width 0.5) (layer "F.Cu") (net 22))
 (via (at 179.5 116) (size 0.6) (drill 0.3) (layers "F.Cu" "B.Cu") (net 22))
 (segment (start 179.5 116) (end 166.81 116) (width 0.5) (layer "B.Cu") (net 22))
 (segment (start 166.81 116) (end 154.42 103.61) (width 0.5) (layer "B.Cu") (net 22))
 (segment (start 167.12 108.18) (end 154.42 120.88) (width 0.5) (layer "F.Cu") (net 10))
 (segment (start 154.42 120.88) (end 154.42 122.66) (width 0.5) (layer "F.Cu") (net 10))
 (segment (start 174.9 121) (end 178.9 121) (width 1) (layer "F.Cu") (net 21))
 (segment (start 174.9 121) (end 174.9 117.9) (width 0.5) (layer "F.Cu") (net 21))
 (segment (start 174.9 117.9) (end 174.5 117.5) (width 0.5) (layer "F.Cu") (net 21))
 (via (at 174.5 117.5) (size 0.6) (drill 0.3) (layers "F.Cu" "B.Cu") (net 21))
 (segment (start 165.146 117.5) (end 151.88 104.234) (width 0.5) (layer "B.Cu") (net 21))
 (segment (start 151.88 104.234) (end 151.88 103.61) (width 1) (layer "B.Cu") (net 21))
 (segment (start 174.5 117.5) (end 165.146 117.5) (width 0.5) (layer "B.Cu") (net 21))
 (segment (start 170.3102 108.9078) (end 170.4078 108.9078) (width 0.2) (layer "F.Cu") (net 5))
 (segment (start 170.4078 108.9078) (end 171 109.5) (width 0.4) (layer "F.Cu") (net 5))
 (segment (start 174.75 105.825) (end 174.625 105.7) (width 0.2) (layer "F.Cu") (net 5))
 (segment (start 174.75 106.75) (end 174.75 105.825) (width 0.2) (layer "F.Cu") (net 5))
 (via (at 174.75 106.75) (size 0.6) (drill 0.3) (layers "F.Cu" "B.Cu") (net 5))
 (via (at 171 109.5) (size 0.6) (drill 0.3) (layers "F.Cu" "B.Cu") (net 5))
 (segment (start 172.25 109.5) (end 174.75 107) (width 0.4) (layer "B.Cu") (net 5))
 (segment (start 174.75 107) (end 174.75 106.75) (width 0.2) (layer "B.Cu") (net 5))
 (segment (start 171 109.5) (end 172.25 109.5) (width 0.4) (layer "B.Cu") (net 5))
 (segment (start 182.5 105.8) (end 182.6 105.7) (width 0.5) (layer "F.Cu") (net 2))
 (segment (start 182.5 108.5) (end 182.5 105.8) (width 0.5) (layer "F.Cu") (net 2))
 (via (at 182.5 108.5) (size 0.6) (drill 0.3) (layers "F.Cu" "B.Cu") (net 2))
 (segment (start 181 110) (end 182.5 108.5) (width 0.5) (layer "B.Cu") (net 2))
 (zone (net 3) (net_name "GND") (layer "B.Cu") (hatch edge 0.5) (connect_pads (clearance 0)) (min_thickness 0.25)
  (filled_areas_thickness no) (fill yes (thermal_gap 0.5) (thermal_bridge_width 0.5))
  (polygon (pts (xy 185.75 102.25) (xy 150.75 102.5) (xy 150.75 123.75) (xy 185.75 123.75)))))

